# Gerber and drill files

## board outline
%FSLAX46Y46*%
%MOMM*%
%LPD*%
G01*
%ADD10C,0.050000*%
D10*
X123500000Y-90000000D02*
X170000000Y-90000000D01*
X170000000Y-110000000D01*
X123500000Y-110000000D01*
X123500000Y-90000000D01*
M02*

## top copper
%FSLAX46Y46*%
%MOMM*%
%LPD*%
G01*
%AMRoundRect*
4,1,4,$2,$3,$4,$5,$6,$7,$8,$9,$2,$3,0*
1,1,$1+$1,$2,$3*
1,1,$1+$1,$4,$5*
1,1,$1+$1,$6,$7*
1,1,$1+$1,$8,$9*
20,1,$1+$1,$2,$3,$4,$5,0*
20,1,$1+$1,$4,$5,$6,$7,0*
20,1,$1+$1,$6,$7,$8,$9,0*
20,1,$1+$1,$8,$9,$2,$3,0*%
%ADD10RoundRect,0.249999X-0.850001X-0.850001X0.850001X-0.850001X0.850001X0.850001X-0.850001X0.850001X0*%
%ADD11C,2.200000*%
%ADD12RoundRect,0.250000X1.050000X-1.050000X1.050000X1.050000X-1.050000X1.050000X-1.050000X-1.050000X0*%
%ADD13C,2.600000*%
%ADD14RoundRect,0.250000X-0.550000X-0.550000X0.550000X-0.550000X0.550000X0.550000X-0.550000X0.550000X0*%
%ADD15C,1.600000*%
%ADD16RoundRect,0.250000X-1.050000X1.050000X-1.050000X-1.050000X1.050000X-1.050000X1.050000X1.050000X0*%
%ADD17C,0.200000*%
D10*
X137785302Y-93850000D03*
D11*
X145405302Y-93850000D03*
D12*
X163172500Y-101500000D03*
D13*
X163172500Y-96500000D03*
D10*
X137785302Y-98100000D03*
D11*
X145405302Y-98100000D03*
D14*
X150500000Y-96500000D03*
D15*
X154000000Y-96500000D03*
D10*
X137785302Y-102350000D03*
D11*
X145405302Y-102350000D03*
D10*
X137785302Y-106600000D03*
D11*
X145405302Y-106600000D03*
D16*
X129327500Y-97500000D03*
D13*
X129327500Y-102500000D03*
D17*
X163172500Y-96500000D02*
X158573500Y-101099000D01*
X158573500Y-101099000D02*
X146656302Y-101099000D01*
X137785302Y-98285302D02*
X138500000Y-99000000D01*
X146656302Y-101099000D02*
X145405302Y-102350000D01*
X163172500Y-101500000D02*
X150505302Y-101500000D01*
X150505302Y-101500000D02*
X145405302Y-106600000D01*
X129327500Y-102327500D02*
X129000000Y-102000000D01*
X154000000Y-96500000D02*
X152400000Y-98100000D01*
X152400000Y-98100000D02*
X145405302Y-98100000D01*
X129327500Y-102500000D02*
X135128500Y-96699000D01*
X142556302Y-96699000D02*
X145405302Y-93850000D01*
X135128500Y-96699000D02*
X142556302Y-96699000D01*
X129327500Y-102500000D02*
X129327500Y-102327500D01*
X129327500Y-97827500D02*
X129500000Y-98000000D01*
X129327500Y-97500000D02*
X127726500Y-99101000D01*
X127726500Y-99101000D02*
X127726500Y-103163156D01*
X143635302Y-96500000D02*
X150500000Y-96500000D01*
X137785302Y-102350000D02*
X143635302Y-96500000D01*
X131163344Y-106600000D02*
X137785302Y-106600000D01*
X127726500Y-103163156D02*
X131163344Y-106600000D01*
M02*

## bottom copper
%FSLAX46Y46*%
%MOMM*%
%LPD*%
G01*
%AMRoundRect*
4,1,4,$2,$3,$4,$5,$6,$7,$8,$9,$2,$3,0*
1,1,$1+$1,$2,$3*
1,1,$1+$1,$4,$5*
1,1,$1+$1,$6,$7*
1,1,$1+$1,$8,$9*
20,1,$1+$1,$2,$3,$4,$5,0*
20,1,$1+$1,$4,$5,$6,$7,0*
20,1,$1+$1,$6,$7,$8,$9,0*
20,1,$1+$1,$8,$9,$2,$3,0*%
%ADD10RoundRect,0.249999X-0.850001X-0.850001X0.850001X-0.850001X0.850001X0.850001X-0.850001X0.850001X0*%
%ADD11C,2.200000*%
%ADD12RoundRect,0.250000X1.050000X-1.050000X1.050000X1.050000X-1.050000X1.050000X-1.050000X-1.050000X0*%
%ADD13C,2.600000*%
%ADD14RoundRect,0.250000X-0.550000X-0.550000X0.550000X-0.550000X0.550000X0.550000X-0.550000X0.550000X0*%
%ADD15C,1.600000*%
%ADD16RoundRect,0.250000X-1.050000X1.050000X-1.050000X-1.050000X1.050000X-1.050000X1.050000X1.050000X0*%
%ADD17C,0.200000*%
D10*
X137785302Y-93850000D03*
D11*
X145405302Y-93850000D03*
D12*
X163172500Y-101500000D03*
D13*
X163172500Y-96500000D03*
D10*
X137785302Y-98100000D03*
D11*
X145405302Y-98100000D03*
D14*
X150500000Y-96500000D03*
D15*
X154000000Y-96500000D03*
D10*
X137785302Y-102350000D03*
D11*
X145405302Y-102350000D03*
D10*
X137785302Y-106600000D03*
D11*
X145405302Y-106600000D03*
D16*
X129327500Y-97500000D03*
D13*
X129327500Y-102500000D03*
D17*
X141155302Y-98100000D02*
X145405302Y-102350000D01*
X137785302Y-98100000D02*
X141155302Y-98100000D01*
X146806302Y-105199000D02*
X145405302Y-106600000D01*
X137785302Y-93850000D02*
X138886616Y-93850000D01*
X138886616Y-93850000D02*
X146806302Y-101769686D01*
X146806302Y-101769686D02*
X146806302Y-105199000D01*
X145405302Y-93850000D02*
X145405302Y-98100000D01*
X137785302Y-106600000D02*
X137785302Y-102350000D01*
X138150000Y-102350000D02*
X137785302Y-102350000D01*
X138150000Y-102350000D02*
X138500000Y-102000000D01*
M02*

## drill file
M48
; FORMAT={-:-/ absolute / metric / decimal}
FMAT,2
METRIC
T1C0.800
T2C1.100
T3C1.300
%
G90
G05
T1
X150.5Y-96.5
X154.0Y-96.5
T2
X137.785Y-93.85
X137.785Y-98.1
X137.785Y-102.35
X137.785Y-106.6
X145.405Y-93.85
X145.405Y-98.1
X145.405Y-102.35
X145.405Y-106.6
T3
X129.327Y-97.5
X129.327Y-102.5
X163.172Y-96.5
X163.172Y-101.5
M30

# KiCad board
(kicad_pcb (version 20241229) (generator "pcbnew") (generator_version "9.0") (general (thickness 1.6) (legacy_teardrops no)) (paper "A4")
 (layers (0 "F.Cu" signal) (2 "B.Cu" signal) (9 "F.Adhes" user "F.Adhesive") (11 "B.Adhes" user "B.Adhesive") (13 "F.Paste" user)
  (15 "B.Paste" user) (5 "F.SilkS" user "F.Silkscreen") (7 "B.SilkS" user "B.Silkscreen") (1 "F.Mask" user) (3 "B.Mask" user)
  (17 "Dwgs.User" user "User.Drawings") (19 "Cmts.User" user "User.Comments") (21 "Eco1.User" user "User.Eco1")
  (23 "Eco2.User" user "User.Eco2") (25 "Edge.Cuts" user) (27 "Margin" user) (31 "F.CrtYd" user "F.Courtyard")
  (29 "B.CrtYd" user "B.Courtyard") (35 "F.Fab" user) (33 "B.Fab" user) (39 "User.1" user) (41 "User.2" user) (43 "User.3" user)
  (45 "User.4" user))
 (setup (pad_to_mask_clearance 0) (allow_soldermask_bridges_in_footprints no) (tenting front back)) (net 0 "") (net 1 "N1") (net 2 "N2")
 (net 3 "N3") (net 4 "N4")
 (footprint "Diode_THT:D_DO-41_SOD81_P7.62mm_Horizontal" (layer "F.Cu") (at 137.785302 93.85)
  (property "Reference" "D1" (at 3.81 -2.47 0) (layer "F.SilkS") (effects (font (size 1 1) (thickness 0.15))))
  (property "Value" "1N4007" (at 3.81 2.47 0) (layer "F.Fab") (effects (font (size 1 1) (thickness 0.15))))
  (pad "1" thru_hole roundrect (at 0 0) (size 2.2 2.2) (drill 1.1) (layers "*.Cu" "*.Mask") (remove_unused_layers no)
   (roundrect_rratio 0.113636) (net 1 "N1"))
  (pad "2" thru_hole circle (at 7.62 0) (size 2.2 2.2) (drill 1.1) (layers "*.Cu" "*.Mask") (remove_unused_layers no) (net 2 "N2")))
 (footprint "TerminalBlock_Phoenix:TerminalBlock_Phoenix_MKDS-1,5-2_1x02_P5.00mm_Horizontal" (layer "F.Cu") (at 163.1725 101.5 90)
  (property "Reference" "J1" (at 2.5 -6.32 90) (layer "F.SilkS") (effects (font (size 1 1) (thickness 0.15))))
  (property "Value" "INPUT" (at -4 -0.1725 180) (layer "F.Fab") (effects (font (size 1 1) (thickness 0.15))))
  (pad "1" thru_hole roundrect (at 0 0 90) (size 2.6 2.6) (drill 1.3) (layers "*.Cu" "*.Mask") (remove_unused_layers no)
   (roundrect_rratio 0.096154) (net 1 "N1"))
  (pad "2" thru_hole circle (at 5 0 90) (size 2.6 2.6) (drill 1.3) (layers "*.Cu" "*.Mask") (remove_unused_layers no) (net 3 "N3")))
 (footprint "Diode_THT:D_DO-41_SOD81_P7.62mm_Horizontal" (layer "F.Cu") (at 137.785302 98.1)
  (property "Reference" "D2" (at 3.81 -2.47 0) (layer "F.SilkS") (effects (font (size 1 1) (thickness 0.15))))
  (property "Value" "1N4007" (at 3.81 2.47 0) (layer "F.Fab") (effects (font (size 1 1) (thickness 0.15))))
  (pad "1" thru_hole roundrect (at 0 0) (size 2.2 2.2) (drill 1.1) (layers "*.Cu" "*.Mask") (remove_unused_layers no)
   (roundrect_rratio 0.113636) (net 3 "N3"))
  (pad "2" thru_hole circle (at 7.62 0) (size 2.2 2.2) (drill 1.1) (layers "*.Cu" "*.Mask") (remove_unused_layers no) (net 2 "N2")))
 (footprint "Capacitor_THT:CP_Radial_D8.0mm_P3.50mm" (layer "F.Cu") (at 150.5 96.5)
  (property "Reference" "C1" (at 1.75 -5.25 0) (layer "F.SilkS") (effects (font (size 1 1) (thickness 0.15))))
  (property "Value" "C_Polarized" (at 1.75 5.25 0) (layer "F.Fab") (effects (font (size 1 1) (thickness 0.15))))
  (pad "1" thru_hole roundrect (at 0 0) (size 1.6 1.6) (drill 0.8) (layers "*.Cu" "*.Mask") (remove_unused_layers no)
   (roundrect_rratio 0.15625) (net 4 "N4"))
  (pad "2" thru_hole circle (at 3.5 0) (size 1.6 1.6) (drill 0.8) (layers "*.Cu" "*.Mask") (remove_unused_layers no) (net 2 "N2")))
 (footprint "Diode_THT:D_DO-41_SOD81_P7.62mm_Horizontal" (layer "F.Cu") (at 137.785302 102.35)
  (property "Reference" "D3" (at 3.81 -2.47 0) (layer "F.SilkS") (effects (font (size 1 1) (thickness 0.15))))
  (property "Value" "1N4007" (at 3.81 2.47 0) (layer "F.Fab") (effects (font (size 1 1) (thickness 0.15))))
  (pad "1" thru_hole roundrect (at 0 0) (size 2.2 2.2) (drill 1.1) (layers "*.Cu" "*.Mask") (remove_unused_layers no)
   (roundrect_rratio 0.113636) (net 4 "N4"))
  (pad "2" thru_hole circle (at 7.62 0) (size 2.2 2.2) (drill 1.1) (layers "*.Cu" "*.Mask") (remove_unused_layers no) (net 3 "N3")))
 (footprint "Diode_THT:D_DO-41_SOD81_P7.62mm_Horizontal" (layer "F.Cu") (at 137.785302 106.6)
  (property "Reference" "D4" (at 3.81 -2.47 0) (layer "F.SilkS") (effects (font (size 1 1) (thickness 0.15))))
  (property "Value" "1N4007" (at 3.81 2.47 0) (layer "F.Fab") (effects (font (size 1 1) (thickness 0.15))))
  (pad "1" thru_hole roundrect (at 0 0) (size 2.2 2.2) (drill 1.1) (layers "*.Cu" "*.Mask") (remove_unused_layers no)
   (roundrect_rratio 0.113636) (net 4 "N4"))
  (pad "2" thru_hole circle (at 7.62 0) (size 2.2 2.2) (drill 1.1) (layers "*.Cu" "*.Mask") (remove_unused_layers no) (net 1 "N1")))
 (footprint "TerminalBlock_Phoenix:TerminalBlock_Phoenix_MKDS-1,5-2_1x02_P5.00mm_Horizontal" (layer "F.Cu") (at 129.3275 97.5 -90)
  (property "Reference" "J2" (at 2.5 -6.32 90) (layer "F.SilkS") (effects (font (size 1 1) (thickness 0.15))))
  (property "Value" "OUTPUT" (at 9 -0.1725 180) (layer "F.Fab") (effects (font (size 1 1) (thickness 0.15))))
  (pad "1" thru_hole roundrect (at 0 0 270) (size 2.6 2.6) (drill 1.3) (layers "*.Cu" "*.Mask") (remove_unused_layers no)
   (roundrect_rratio 0.096154) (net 4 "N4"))
  (pad "2" thru_hole circle (at 5 0 270) (size 2.6 2.6) (drill 1.3) (layers "*.Cu" "*.Mask") (remove_unused_layers no) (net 2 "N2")))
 (gr_rect (start 123.5 90) (end 170 110) (stroke (width 0.05) (type default)) (fill no) (layer "Edge.Cuts"))
 (segment (start 163.1725 96.5) (end 158.5735 101.099) (width 0.2) (layer "F.Cu") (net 3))
 (segment (start 158.5735 101.099) (end 146.656302 101.099) (width 0.2) (layer "F.Cu") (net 3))
 (segment (start 137.785302 98.285302) (end 138.5 99) (width 0.2) (layer "F.Cu") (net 3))
 (segment (start 146.656302 101.099) (end 145.405302 102.35) (width 0.2) (layer "F.Cu") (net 3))
 (segment (start 141.155302 98.1) (end 145.405302 102.35) (width 0.2) (layer "B.Cu") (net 3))
 (segment (start 137.785302 98.1) (end 141.155302 98.1) (width 0.2) (layer "B.Cu") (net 3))
 (segment (start 163.1725 101.5) (end 150.505302 101.5) (width 0.2) (layer "F.Cu") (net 1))
 (segment (start 150.505302 101.5) (end 145.405302 106.6) (width 0.2) (layer "F.Cu") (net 1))
 (segment (start 146.806302 105.199) (end 145.405302 106.6) (width 0.2) (layer "B.Cu") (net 1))
 (segment (start 137.785302 93.85) (end 138.886616 93.85) (width 0.2) (layer "B.Cu") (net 1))
 (segment (start 138.886616 93.85) (end 146.806302 101.769686) (width 0.2) (layer "B.Cu") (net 1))
 (segment (start 146.806302 101.769686) (end 146.806302 105.199) (width 0.2) (layer "B.Cu") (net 1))
 (segment (start 129.3275 102.3275) (end 129 102) (width 0.2) (layer "F.Cu") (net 2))
 (segment (start 154 96.5) (end 152.4 98.1) (width 0.2) (layer "F.Cu") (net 2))
 (segment (start 152.4 98.1) (end 145.405302 98.1) (width 0.2) (layer "F.Cu") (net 2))
 (segment (start 129.3275 102.5) (end 135.1285 96.699) (width 0.2) (layer "F.Cu") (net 2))
 (segment (start 142.556302 96.699) (end 145.405302 93.85) (width 0.2) (layer "F.Cu") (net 2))
 (segment (start 135.1285 96.699) (end 142.556302 96.699) (width 0.2) (layer "F.Cu") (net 2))
 (segment (start 129.3275 102.5) (end 129.3275 102.3275) (width 0.2) (layer "F.Cu") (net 2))
 (segment (start 145.405302 93.85) (end 145.405302 98.1) (width 0.2) (layer "B.Cu") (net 2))
 (segment (start 129.3275 97.8275) (end 129.5 98) (width 0.2) (layer "F.Cu") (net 4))
 (segment (start 129.3275 97.5) (end 127.7265 99.101) (width 0.2) (layer "F.Cu") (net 4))
 (segment (start 127.7265 99.101) (end 127.7265 103.163156) (width 0.2) (layer "F.Cu") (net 4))
 (segment (start 143.635302 96.5) (end 150.5 96.5) (width 0.2) (layer "F.Cu") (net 4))
 (segment (start 137.785302 102.35) (end 143.635302 96.5) (width 0.2) (layer "F.Cu") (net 4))
 (segment (start 131.163344 106.6) (end 137.785302 106.6) (width 0.2) (layer "F.Cu") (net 4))
 (segment (start 127.7265 103.163156) (end 131.163344 106.6) (width 0.2) (layer "F.Cu") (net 4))
 (segment (start 137.785302 106.6) (end 137.785302 102.35) (width 0.2) (layer "B.Cu") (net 4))
 (segment (start 138.15 102.35) (end 137.785302 102.35) (width 0.2) (layer "B.Cu") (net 4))
 (segment (start 138.15 102.35) (end 138.5 102) (width 0.2) (layer "B.Cu") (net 4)))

